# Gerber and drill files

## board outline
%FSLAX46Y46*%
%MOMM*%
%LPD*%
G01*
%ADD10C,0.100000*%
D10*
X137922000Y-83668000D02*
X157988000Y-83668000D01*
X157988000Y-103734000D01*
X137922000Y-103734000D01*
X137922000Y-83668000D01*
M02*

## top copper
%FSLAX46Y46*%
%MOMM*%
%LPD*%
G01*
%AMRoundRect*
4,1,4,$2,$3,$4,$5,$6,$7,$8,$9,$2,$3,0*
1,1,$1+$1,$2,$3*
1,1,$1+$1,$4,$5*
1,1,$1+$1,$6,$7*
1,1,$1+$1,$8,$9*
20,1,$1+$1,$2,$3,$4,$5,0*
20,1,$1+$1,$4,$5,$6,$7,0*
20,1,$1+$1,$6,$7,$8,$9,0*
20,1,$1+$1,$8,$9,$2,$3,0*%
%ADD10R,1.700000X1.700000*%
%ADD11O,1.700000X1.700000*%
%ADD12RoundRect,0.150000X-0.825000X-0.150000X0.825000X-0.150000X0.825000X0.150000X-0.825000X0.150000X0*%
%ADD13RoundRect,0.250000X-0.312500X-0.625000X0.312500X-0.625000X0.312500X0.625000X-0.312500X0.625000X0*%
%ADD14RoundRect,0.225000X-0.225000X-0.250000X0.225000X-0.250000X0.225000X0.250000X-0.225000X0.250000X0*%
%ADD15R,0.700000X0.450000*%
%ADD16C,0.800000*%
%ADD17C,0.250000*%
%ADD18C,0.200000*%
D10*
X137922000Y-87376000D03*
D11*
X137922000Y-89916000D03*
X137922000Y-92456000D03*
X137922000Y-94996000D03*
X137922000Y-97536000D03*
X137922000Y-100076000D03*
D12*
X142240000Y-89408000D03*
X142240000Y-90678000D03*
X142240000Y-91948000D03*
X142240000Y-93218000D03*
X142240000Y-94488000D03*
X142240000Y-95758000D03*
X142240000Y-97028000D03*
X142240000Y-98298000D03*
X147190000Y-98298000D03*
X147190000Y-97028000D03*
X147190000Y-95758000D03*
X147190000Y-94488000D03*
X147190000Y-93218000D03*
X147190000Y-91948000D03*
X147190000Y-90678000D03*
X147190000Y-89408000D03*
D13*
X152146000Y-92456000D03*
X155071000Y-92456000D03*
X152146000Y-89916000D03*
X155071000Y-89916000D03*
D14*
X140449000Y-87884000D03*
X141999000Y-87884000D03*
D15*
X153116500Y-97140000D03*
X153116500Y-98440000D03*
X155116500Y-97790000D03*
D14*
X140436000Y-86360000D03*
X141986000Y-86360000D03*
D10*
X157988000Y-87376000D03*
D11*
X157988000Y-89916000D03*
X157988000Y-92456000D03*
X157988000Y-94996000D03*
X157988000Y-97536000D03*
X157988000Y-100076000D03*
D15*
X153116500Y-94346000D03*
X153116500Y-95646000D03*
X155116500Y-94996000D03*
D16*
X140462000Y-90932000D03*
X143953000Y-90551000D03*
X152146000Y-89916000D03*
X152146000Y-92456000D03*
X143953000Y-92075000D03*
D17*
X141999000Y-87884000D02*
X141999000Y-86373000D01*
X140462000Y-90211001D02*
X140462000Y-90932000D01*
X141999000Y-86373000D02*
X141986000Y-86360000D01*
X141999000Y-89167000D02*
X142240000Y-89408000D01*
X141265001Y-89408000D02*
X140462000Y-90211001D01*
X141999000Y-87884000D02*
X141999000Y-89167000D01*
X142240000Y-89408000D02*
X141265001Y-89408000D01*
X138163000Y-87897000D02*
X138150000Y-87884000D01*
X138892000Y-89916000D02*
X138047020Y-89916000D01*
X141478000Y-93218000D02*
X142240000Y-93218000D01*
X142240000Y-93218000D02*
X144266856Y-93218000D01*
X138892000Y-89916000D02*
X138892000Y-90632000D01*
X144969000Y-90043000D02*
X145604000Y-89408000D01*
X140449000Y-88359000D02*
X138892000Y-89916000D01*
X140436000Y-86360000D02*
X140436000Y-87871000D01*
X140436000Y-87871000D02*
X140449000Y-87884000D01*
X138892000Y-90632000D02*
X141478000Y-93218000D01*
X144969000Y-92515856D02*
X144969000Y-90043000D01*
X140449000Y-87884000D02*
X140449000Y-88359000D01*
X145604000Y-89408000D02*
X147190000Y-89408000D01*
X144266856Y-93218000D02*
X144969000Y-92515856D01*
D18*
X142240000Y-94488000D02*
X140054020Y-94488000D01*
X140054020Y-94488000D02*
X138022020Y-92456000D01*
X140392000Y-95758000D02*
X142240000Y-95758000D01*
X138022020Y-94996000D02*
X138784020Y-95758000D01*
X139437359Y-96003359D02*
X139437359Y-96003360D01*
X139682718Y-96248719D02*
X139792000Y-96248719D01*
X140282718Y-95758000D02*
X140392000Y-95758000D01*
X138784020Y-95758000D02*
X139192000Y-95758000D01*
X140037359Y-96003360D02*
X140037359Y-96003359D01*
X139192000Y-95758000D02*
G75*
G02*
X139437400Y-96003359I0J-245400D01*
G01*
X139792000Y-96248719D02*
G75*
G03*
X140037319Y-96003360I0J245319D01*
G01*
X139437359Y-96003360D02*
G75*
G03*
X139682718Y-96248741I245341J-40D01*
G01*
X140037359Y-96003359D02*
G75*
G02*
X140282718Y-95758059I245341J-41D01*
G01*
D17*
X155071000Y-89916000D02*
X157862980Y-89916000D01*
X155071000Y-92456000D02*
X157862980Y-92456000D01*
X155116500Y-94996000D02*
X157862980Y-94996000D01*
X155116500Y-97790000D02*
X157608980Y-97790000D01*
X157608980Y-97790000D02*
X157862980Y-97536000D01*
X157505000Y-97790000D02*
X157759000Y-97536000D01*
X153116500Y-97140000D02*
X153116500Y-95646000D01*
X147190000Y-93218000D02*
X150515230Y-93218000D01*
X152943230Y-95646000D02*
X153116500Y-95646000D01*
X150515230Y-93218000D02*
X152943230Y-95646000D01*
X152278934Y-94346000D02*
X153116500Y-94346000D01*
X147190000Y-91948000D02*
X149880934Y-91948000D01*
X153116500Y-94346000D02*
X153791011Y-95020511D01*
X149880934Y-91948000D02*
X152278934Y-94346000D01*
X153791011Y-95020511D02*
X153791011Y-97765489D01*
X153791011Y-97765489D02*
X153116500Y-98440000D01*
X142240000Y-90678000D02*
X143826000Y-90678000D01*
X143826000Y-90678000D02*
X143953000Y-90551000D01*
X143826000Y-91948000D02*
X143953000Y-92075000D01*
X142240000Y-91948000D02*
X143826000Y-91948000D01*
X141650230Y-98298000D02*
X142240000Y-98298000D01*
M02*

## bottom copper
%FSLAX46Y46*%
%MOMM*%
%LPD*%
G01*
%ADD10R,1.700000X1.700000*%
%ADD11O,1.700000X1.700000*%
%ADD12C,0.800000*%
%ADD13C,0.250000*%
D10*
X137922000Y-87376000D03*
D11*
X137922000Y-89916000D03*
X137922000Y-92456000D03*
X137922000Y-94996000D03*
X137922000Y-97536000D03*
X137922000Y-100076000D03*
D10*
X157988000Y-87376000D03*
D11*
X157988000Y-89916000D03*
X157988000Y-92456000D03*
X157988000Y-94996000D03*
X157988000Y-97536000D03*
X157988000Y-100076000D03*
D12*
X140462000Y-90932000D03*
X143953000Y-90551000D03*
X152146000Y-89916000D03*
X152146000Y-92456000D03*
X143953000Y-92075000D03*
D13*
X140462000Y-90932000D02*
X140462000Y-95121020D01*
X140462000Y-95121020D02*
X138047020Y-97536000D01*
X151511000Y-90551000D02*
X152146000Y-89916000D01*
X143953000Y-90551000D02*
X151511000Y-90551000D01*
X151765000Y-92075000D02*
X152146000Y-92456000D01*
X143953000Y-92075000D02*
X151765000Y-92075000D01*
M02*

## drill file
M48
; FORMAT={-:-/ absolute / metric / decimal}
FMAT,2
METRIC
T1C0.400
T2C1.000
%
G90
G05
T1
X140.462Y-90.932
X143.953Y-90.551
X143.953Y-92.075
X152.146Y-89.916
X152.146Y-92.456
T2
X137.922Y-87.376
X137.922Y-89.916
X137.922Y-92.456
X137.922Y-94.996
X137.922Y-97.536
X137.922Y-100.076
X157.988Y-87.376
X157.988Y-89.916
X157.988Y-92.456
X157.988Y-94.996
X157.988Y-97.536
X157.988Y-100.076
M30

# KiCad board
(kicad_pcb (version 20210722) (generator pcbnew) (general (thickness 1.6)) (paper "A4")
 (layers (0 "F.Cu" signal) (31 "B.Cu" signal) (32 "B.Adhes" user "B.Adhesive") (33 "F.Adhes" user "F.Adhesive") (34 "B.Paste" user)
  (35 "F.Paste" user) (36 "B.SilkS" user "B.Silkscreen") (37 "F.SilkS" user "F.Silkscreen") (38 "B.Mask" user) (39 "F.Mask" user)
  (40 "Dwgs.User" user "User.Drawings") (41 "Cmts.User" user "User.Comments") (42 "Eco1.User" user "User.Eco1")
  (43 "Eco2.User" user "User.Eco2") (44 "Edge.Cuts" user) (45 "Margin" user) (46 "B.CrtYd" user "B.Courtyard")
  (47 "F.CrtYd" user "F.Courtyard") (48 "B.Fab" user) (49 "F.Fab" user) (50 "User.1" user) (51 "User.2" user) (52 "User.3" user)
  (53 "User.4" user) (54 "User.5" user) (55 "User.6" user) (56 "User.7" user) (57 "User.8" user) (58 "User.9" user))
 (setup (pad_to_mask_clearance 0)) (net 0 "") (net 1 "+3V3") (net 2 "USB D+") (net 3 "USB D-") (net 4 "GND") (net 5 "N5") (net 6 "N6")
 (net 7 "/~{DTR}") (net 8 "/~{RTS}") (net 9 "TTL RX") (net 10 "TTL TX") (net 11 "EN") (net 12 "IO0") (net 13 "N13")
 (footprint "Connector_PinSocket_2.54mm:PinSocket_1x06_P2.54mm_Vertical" (layer "F.Cu") (at 137.922 87.376)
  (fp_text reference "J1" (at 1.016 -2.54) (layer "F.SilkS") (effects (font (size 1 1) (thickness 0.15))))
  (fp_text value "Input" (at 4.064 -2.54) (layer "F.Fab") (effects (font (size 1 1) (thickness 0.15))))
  (pad "1" thru_hole rect locked (at 0 0) (size 1.7 1.7) (drill 1) (layers *.Cu *.Mask))
  (pad "2" thru_hole oval locked (at 0 2.54) (size 1.7 1.7) (drill 1) (layers *.Cu *.Mask) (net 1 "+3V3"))
  (pad "3" thru_hole oval locked (at 0 5.08) (size 1.7 1.7) (drill 1) (layers *.Cu *.Mask) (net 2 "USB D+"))
  (pad "4" thru_hole oval locked (at 0 7.62) (size 1.7 1.7) (drill 1) (layers *.Cu *.Mask) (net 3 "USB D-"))
  (pad "5" thru_hole oval locked (at 0 10.16) (size 1.7 1.7) (drill 1) (layers *.Cu *.Mask) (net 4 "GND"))
  (pad "6" thru_hole oval locked (at 0 12.7) (size 1.7 1.7) (drill 1) (layers *.Cu *.Mask)))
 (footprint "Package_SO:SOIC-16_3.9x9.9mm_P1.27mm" (layer "F.Cu") (at 144.715 93.853)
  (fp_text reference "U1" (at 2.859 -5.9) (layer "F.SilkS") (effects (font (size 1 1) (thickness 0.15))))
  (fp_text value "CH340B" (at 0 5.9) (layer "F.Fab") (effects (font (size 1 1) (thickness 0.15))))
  (pad "1" smd roundrect locked (at -2.475 -4.445) (size 1.95 0.6) (layers "F.Cu" "F.Paste" "F.Mask") (roundrect_rratio 0.25) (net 4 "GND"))
  (pad "2" smd roundrect locked (at -2.475 -3.175) (size 1.95 0.6) (layers "F.Cu" "F.Paste" "F.Mask") (roundrect_rratio 0.25) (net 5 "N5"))
  (pad "3" smd roundrect locked (at -2.475 -1.905) (size 1.95 0.6) (layers "F.Cu" "F.Paste" "F.Mask") (roundrect_rratio 0.25) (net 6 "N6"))
  (pad "4" smd roundrect locked (at -2.475 -0.635) (size 1.95 0.6) (layers "F.Cu" "F.Paste" "F.Mask") (roundrect_rratio 0.25) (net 1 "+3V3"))
  (pad "5" smd roundrect locked (at -2.475 0.635) (size 1.95 0.6) (layers "F.Cu" "F.Paste" "F.Mask") (roundrect_rratio 0.25)
   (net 2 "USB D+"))
  (pad "6" smd roundrect locked (at -2.475 1.905) (size 1.95 0.6) (layers "F.Cu" "F.Paste" "F.Mask") (roundrect_rratio 0.25)
   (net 3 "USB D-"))
  (pad "7" smd roundrect locked (at -2.475 3.175) (size 1.95 0.6) (layers "F.Cu" "F.Paste" "F.Mask") (roundrect_rratio 0.25))
  (pad "8" smd roundrect locked (at -2.475 4.445) (size 1.95 0.6) (layers "F.Cu" "F.Paste" "F.Mask") (roundrect_rratio 0.25))
  (pad "9" smd roundrect locked (at 2.475 4.445) (size 1.95 0.6) (layers "F.Cu" "F.Paste" "F.Mask") (roundrect_rratio 0.25))
  (pad "10" smd roundrect locked (at 2.475 3.175) (size 1.95 0.6) (layers "F.Cu" "F.Paste" "F.Mask") (roundrect_rratio 0.25))
  (pad "11" smd roundrect locked (at 2.475 1.905) (size 1.95 0.6) (layers "F.Cu" "F.Paste" "F.Mask") (roundrect_rratio 0.25))
  (pad "12" smd roundrect locked (at 2.475 0.635) (size 1.95 0.6) (layers "F.Cu" "F.Paste" "F.Mask") (roundrect_rratio 0.25))
  (pad "13" smd roundrect locked (at 2.475 -0.635) (size 1.95 0.6) (layers "F.Cu" "F.Paste" "F.Mask") (roundrect_rratio 0.25)
   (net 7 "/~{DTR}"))
  (pad "14" smd roundrect locked (at 2.475 -1.905) (size 1.95 0.6) (layers "F.Cu" "F.Paste" "F.Mask") (roundrect_rratio 0.25)
   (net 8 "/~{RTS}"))
  (pad "15" smd roundrect locked (at 2.475 -3.175) (size 1.95 0.6) (layers "F.Cu" "F.Paste" "F.Mask") (roundrect_rratio 0.25))
  (pad "16" smd roundrect locked (at 2.475 -4.445) (size 1.95 0.6) (layers "F.Cu" "F.Paste" "F.Mask") (roundrect_rratio 0.25) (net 1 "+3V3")))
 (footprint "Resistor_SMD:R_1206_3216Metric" (layer "F.Cu") (at 153.6085 92.456)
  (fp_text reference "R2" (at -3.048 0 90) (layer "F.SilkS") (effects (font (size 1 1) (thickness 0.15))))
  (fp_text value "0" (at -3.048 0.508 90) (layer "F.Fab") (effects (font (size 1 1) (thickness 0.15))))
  (pad "1" smd roundrect locked (at -1.4625 0) (size 1.125 1.75) (layers "F.Cu" "F.Paste" "F.Mask") (roundrect_rratio 0.222222) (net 6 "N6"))
  (pad "2" smd roundrect locked (at 1.4625 0) (size 1.125 1.75) (layers "F.Cu" "F.Paste" "F.Mask") (roundrect_rratio 0.222222)
   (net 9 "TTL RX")))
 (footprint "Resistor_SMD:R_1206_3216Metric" (layer "F.Cu") (at 153.6085 89.916)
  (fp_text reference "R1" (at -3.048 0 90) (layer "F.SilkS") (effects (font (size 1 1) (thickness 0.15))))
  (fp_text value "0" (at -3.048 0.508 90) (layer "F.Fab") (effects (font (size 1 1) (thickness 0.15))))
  (pad "1" smd roundrect locked (at -1.4625 0) (size 1.125 1.75) (layers "F.Cu" "F.Paste" "F.Mask") (roundrect_rratio 0.222222) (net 5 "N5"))
  (pad "2" smd roundrect locked (at 1.4625 0) (size 1.125 1.75) (layers "F.Cu" "F.Paste" "F.Mask") (roundrect_rratio 0.222222)
   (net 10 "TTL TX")))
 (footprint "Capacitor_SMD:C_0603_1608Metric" (layer "F.Cu") (at 141.224 87.884)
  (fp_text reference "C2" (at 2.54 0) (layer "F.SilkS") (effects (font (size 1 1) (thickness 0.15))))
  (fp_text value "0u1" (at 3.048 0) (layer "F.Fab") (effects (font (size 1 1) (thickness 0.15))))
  (pad "1" smd roundrect locked (at -0.775 0) (size 0.9 0.95) (layers "F.Cu" "F.Paste" "F.Mask") (roundrect_rratio 0.25) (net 1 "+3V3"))
  (pad "2" smd roundrect locked (at 0.775 0) (size 0.9 0.95) (layers "F.Cu" "F.Paste" "F.Mask") (roundrect_rratio 0.25) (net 4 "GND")))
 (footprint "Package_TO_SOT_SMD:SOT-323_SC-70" (layer "F.Cu") (at 154.1165 97.79)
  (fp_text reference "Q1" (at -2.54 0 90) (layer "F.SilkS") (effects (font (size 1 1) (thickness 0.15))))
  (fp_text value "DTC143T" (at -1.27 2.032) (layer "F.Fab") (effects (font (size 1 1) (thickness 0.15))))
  (pad "1" smd rect locked (at -1 -0.65 270) (size 0.45 0.7) (layers "F.Cu" "F.Paste" "F.Mask") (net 7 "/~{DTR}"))
  (pad "2" smd rect locked (at -1 0.65 270) (size 0.45 0.7) (layers "F.Cu" "F.Paste" "F.Mask") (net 8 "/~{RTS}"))
  (pad "3" smd rect locked (at 1 0 270) (size 0.45 0.7) (layers "F.Cu" "F.Paste" "F.Mask") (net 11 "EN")))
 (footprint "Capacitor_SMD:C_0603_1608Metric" (layer "F.Cu") (at 141.211 86.36)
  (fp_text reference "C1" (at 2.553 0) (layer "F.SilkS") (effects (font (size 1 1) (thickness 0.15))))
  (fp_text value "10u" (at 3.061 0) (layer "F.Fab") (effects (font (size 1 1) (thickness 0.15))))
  (pad "1" smd roundrect locked (at -0.775 0) (size 0.9 0.95) (layers "F.Cu" "F.Paste" "F.Mask") (roundrect_rratio 0.25) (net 1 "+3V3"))
  (pad "2" smd roundrect locked (at 0.775 0) (size 0.9 0.95) (layers "F.Cu" "F.Paste" "F.Mask") (roundrect_rratio 0.25) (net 4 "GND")))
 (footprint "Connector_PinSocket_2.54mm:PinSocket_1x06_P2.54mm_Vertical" (layer "F.Cu") (at 157.988 87.376)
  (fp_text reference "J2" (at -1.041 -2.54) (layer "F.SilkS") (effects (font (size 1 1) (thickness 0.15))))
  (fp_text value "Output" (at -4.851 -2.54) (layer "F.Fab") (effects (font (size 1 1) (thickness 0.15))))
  (pad "1" thru_hole rect locked (at 0 0) (size 1.7 1.7) (drill 1) (layers *.Cu *.Mask))
  (pad "2" thru_hole oval locked (at 0 2.54) (size 1.7 1.7) (drill 1) (layers *.Cu *.Mask) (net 10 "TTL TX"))
  (pad "3" thru_hole oval locked (at 0 5.08) (size 1.7 1.7) (drill 1) (layers *.Cu *.Mask) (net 9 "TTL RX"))
  (pad "4" thru_hole oval locked (at 0 7.62) (size 1.7 1.7) (drill 1) (layers *.Cu *.Mask) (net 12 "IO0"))
  (pad "5" thru_hole oval locked (at 0 10.16) (size 1.7 1.7) (drill 1) (layers *.Cu *.Mask) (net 11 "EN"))
  (pad "6" thru_hole oval locked (at 0 12.7) (size 1.7 1.7) (drill 1) (layers *.Cu *.Mask)))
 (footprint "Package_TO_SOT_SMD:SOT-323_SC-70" (layer "F.Cu") (at 154.1165 94.996)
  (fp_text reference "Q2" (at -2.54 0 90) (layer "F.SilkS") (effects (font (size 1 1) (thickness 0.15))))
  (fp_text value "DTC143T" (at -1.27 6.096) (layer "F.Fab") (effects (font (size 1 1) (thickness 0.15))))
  (pad "1" smd rect locked (at -1 -0.65 270) (size 0.45 0.7) (layers "F.Cu" "F.Paste" "F.Mask") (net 8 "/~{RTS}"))
  (pad "2" smd rect locked (at -1 0.65 270) (size 0.45 0.7) (layers "F.Cu" "F.Paste" "F.Mask") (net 7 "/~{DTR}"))
  (pad "3" smd rect locked (at 1 0 270) (size 0.45 0.7) (layers "F.Cu" "F.Paste" "F.Mask") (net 12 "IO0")))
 (gr_rect (start 157.988 103.734) (end 137.922 83.668) (layer "Edge.Cuts") (width 0.1) (fill none))
 (segment (start 141.999 87.884) (end 141.999 86.373) (width 0.25) (layer "F.Cu") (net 4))
 (segment (start 140.462 90.211001) (end 140.462 90.932) (width 0.25) (layer "F.Cu") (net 4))
 (segment (start 141.999 86.373) (end 141.986 86.36) (width 0.25) (layer "F.Cu") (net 4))
 (segment (start 141.999 89.167) (end 142.24 89.408) (width 0.25) (layer "F.Cu") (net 4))
 (segment (start 141.265001 89.408) (end 140.462 90.211001) (width 0.25) (layer "F.Cu") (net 4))
 (segment (start 141.999 87.884) (end 141.999 89.167) (width 0.25) (layer "F.Cu") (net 4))
 (segment (start 142.24 89.408) (end 141.265001 89.408) (width 0.25) (layer "F.Cu") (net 4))
 (via (at 140.462 90.932) (size 0.8) (drill 0.4) (layers "F.Cu" "B.Cu") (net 4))
 (segment (start 140.462 90.932) (end 140.462 95.12102) (width 0.25) (layer "B.Cu") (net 4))
 (segment (start 140.462 95.12102) (end 138.04702 97.536) (width 0.25) (layer "B.Cu") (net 4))
 (segment (start 138.163 87.897) (end 138.15 87.884) (width 0.25) (layer "F.Cu") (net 1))
 (segment (start 138.892 89.916) (end 138.04702 89.916) (width 0.25) (layer "F.Cu") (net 1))
 (segment (start 141.478 93.218) (end 142.24 93.218) (width 0.25) (layer "F.Cu") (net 1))
 (segment (start 142.24 93.218) (end 144.266856 93.218) (width 0.25) (layer "F.Cu") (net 1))
 (segment (start 138.892 89.916) (end 138.892 90.632) (width 0.25) (layer "F.Cu") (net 1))
 (segment (start 144.969 90.043) (end 145.604 89.408) (width 0.25) (layer "F.Cu") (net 1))
 (segment (start 140.449 88.359) (end 138.892 89.916) (width 0.25) (layer "F.Cu") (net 1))
 (segment (start 140.436 86.36) (end 140.436 87.871) (width 0.25) (layer "F.Cu") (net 1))
 (segment (start 140.436 87.871) (end 140.449 87.884) (width 0.25) (layer "F.Cu") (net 1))
 (segment (start 138.892 90.632) (end 141.478 93.218) (width 0.25) (layer "F.Cu") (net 1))
 (segment (start 144.969 92.515856) (end 144.969 90.043) (width 0.25) (layer "F.Cu") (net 1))
 (segment (start 140.449 87.884) (end 140.449 88.359) (width 0.25) (layer "F.Cu") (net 1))
 (segment (start 145.604 89.408) (end 147.19 89.408) (width 0.25) (layer "F.Cu") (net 1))
 (segment (start 144.266856 93.218) (end 144.969 92.515856) (width 0.25) (layer "F.Cu") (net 1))
 (segment (start 142.24 94.488) (end 140.05402 94.488) (width 0.2) (layer "F.Cu") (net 2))
 (segment (start 140.05402 94.488) (end 138.02202 92.456) (width 0.2) (layer "F.Cu") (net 2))
 (segment (start 140.392 95.758) (end 142.24 95.758) (width 0.2) (layer "F.Cu") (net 3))
 (segment (start 138.02202 94.996) (end 138.78402 95.758) (width 0.2) (layer "F.Cu") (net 3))
 (segment (start 139.437359 96.003359) (end 139.437359 96.00336) (width 0.2) (layer "F.Cu") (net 3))
 (segment (start 139.682718 96.248719) (end 139.792 96.248719) (width 0.2) (layer "F.Cu") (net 3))
 (segment (start 140.282718 95.758) (end 140.392 95.758) (width 0.2) (layer "F.Cu") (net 3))
 (segment (start 138.78402 95.758) (end 139.192 95.758) (width 0.2) (layer "F.Cu") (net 3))
 (segment (start 140.037359 96.00336) (end 140.037359 96.003359) (width 0.2) (layer "F.Cu") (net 3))
 (arc (start 139.192 95.758) (mid 139.365495 95.829864) (end 139.437359 96.003359) (width 0.2) (layer "F.Cu") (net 3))
 (arc (start 139.792 96.248719) (mid 139.965495 96.176855) (end 140.037359 96.00336) (width 0.2) (layer "F.Cu") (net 3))
 (arc (start 139.437359 96.00336) (mid 139.509223 96.176855) (end 139.682718 96.248719) (width 0.2) (layer "F.Cu") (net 3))
 (arc (start 140.037359 96.003359) (mid 140.109223 95.829864) (end 140.282718 95.758) (width 0.2) (layer "F.Cu") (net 3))
 (segment (start 155.071 89.916) (end 157.86298 89.916) (width 0.25) (layer "F.Cu") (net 10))
 (segment (start 155.071 92.456) (end 157.86298 92.456) (width 0.25) (layer "F.Cu") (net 9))
 (segment (start 155.1165 94.996) (end 157.86298 94.996) (width 0.25) (layer "F.Cu") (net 12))
 (segment (start 155.1165 97.79) (end 157.60898 97.79) (width 0.25) (layer "F.Cu") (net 11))
 (segment (start 157.60898 97.79) (end 157.86298 97.536) (width 0.25) (layer "F.Cu") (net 11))
 (segment (start 157.505 97.79) (end 157.759 97.536) (width 0.25) (layer "F.Cu") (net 11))
 (segment (start 153.1165 97.14) (end 153.1165 95.646) (width 0.25) (layer "F.Cu") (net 7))
 (segment (start 147.19 93.218) (end 150.51523 93.218) (width 0.25) (layer "F.Cu") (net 7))
 (segment (start 152.94323 95.646) (end 153.1165 95.646) (width 0.25) (layer "F.Cu") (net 7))
 (segment (start 150.51523 93.218) (end 152.94323 95.646) (width 0.25) (layer "F.Cu") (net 7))
 (segment (start 152.278934 94.346) (end 153.1165 94.346) (width 0.25) (layer "F.Cu") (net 8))
 (segment (start 147.19 91.948) (end 149.880934 91.948) (width 0.25) (layer "F.Cu") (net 8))
 (segment (start 153.1165 94.346) (end 153.791011 95.020511) (width 0.25) (layer "F.Cu") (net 8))
 (segment (start 149.880934 91.948) (end 152.278934 94.346) (width 0.25) (layer "F.Cu") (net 8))
 (segment (start 153.791011 95.020511) (end 153.791011 97.765489) (width 0.25) (layer "F.Cu") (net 8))
 (segment (start 153.791011 97.765489) (end 153.1165 98.44) (width 0.25) (layer "F.Cu") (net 8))
 (segment (start 142.24 90.678) (end 143.826 90.678) (width 0.25) (layer "F.Cu") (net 5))
 (segment (start 143.826 90.678) (end 143.953 90.551) (width 0.25) (layer "F.Cu") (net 5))
 (via (at 143.953 90.551) (size 0.8) (drill 0.4) (layers "F.Cu" "B.Cu") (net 5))
 (via (at 152.146 89.916) (size 0.8) (drill 0.4) (layers "F.Cu" "B.Cu") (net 5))
 (segment (start 151.511 90.551) (end 152.146 89.916) (width 0.25) (layer "B.Cu") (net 5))
 (segment (start 143.953 90.551) (end 151.511 90.551) (width 0.25) (layer "B.Cu") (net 5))
 (segment (start 143.826 91.948) (end 143.953 92.075) (width 0.25) (layer "F.Cu") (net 6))
 (segment (start 142.24 91.948) (end 143.826 91.948) (width 0.25) (layer "F.Cu") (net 6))
 (via (at 152.146 92.456) (size 0.8) (drill 0.4) (layers "F.Cu" "B.Cu") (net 6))
 (via (at 143.953 92.075) (size 0.8) (drill 0.4) (layers "F.Cu" "B.Cu") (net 6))
 (segment (start 151.765 92.075) (end 152.146 92.456) (width 0.25) (layer "B.Cu") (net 6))
 (segment (start 143.953 92.075) (end 151.765 92.075) (width 0.25) (layer "B.Cu") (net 6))
 (segment (start 141.65023 98.298) (end 142.24 98.298) (width 0.25) (layer "F.Cu") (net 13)))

